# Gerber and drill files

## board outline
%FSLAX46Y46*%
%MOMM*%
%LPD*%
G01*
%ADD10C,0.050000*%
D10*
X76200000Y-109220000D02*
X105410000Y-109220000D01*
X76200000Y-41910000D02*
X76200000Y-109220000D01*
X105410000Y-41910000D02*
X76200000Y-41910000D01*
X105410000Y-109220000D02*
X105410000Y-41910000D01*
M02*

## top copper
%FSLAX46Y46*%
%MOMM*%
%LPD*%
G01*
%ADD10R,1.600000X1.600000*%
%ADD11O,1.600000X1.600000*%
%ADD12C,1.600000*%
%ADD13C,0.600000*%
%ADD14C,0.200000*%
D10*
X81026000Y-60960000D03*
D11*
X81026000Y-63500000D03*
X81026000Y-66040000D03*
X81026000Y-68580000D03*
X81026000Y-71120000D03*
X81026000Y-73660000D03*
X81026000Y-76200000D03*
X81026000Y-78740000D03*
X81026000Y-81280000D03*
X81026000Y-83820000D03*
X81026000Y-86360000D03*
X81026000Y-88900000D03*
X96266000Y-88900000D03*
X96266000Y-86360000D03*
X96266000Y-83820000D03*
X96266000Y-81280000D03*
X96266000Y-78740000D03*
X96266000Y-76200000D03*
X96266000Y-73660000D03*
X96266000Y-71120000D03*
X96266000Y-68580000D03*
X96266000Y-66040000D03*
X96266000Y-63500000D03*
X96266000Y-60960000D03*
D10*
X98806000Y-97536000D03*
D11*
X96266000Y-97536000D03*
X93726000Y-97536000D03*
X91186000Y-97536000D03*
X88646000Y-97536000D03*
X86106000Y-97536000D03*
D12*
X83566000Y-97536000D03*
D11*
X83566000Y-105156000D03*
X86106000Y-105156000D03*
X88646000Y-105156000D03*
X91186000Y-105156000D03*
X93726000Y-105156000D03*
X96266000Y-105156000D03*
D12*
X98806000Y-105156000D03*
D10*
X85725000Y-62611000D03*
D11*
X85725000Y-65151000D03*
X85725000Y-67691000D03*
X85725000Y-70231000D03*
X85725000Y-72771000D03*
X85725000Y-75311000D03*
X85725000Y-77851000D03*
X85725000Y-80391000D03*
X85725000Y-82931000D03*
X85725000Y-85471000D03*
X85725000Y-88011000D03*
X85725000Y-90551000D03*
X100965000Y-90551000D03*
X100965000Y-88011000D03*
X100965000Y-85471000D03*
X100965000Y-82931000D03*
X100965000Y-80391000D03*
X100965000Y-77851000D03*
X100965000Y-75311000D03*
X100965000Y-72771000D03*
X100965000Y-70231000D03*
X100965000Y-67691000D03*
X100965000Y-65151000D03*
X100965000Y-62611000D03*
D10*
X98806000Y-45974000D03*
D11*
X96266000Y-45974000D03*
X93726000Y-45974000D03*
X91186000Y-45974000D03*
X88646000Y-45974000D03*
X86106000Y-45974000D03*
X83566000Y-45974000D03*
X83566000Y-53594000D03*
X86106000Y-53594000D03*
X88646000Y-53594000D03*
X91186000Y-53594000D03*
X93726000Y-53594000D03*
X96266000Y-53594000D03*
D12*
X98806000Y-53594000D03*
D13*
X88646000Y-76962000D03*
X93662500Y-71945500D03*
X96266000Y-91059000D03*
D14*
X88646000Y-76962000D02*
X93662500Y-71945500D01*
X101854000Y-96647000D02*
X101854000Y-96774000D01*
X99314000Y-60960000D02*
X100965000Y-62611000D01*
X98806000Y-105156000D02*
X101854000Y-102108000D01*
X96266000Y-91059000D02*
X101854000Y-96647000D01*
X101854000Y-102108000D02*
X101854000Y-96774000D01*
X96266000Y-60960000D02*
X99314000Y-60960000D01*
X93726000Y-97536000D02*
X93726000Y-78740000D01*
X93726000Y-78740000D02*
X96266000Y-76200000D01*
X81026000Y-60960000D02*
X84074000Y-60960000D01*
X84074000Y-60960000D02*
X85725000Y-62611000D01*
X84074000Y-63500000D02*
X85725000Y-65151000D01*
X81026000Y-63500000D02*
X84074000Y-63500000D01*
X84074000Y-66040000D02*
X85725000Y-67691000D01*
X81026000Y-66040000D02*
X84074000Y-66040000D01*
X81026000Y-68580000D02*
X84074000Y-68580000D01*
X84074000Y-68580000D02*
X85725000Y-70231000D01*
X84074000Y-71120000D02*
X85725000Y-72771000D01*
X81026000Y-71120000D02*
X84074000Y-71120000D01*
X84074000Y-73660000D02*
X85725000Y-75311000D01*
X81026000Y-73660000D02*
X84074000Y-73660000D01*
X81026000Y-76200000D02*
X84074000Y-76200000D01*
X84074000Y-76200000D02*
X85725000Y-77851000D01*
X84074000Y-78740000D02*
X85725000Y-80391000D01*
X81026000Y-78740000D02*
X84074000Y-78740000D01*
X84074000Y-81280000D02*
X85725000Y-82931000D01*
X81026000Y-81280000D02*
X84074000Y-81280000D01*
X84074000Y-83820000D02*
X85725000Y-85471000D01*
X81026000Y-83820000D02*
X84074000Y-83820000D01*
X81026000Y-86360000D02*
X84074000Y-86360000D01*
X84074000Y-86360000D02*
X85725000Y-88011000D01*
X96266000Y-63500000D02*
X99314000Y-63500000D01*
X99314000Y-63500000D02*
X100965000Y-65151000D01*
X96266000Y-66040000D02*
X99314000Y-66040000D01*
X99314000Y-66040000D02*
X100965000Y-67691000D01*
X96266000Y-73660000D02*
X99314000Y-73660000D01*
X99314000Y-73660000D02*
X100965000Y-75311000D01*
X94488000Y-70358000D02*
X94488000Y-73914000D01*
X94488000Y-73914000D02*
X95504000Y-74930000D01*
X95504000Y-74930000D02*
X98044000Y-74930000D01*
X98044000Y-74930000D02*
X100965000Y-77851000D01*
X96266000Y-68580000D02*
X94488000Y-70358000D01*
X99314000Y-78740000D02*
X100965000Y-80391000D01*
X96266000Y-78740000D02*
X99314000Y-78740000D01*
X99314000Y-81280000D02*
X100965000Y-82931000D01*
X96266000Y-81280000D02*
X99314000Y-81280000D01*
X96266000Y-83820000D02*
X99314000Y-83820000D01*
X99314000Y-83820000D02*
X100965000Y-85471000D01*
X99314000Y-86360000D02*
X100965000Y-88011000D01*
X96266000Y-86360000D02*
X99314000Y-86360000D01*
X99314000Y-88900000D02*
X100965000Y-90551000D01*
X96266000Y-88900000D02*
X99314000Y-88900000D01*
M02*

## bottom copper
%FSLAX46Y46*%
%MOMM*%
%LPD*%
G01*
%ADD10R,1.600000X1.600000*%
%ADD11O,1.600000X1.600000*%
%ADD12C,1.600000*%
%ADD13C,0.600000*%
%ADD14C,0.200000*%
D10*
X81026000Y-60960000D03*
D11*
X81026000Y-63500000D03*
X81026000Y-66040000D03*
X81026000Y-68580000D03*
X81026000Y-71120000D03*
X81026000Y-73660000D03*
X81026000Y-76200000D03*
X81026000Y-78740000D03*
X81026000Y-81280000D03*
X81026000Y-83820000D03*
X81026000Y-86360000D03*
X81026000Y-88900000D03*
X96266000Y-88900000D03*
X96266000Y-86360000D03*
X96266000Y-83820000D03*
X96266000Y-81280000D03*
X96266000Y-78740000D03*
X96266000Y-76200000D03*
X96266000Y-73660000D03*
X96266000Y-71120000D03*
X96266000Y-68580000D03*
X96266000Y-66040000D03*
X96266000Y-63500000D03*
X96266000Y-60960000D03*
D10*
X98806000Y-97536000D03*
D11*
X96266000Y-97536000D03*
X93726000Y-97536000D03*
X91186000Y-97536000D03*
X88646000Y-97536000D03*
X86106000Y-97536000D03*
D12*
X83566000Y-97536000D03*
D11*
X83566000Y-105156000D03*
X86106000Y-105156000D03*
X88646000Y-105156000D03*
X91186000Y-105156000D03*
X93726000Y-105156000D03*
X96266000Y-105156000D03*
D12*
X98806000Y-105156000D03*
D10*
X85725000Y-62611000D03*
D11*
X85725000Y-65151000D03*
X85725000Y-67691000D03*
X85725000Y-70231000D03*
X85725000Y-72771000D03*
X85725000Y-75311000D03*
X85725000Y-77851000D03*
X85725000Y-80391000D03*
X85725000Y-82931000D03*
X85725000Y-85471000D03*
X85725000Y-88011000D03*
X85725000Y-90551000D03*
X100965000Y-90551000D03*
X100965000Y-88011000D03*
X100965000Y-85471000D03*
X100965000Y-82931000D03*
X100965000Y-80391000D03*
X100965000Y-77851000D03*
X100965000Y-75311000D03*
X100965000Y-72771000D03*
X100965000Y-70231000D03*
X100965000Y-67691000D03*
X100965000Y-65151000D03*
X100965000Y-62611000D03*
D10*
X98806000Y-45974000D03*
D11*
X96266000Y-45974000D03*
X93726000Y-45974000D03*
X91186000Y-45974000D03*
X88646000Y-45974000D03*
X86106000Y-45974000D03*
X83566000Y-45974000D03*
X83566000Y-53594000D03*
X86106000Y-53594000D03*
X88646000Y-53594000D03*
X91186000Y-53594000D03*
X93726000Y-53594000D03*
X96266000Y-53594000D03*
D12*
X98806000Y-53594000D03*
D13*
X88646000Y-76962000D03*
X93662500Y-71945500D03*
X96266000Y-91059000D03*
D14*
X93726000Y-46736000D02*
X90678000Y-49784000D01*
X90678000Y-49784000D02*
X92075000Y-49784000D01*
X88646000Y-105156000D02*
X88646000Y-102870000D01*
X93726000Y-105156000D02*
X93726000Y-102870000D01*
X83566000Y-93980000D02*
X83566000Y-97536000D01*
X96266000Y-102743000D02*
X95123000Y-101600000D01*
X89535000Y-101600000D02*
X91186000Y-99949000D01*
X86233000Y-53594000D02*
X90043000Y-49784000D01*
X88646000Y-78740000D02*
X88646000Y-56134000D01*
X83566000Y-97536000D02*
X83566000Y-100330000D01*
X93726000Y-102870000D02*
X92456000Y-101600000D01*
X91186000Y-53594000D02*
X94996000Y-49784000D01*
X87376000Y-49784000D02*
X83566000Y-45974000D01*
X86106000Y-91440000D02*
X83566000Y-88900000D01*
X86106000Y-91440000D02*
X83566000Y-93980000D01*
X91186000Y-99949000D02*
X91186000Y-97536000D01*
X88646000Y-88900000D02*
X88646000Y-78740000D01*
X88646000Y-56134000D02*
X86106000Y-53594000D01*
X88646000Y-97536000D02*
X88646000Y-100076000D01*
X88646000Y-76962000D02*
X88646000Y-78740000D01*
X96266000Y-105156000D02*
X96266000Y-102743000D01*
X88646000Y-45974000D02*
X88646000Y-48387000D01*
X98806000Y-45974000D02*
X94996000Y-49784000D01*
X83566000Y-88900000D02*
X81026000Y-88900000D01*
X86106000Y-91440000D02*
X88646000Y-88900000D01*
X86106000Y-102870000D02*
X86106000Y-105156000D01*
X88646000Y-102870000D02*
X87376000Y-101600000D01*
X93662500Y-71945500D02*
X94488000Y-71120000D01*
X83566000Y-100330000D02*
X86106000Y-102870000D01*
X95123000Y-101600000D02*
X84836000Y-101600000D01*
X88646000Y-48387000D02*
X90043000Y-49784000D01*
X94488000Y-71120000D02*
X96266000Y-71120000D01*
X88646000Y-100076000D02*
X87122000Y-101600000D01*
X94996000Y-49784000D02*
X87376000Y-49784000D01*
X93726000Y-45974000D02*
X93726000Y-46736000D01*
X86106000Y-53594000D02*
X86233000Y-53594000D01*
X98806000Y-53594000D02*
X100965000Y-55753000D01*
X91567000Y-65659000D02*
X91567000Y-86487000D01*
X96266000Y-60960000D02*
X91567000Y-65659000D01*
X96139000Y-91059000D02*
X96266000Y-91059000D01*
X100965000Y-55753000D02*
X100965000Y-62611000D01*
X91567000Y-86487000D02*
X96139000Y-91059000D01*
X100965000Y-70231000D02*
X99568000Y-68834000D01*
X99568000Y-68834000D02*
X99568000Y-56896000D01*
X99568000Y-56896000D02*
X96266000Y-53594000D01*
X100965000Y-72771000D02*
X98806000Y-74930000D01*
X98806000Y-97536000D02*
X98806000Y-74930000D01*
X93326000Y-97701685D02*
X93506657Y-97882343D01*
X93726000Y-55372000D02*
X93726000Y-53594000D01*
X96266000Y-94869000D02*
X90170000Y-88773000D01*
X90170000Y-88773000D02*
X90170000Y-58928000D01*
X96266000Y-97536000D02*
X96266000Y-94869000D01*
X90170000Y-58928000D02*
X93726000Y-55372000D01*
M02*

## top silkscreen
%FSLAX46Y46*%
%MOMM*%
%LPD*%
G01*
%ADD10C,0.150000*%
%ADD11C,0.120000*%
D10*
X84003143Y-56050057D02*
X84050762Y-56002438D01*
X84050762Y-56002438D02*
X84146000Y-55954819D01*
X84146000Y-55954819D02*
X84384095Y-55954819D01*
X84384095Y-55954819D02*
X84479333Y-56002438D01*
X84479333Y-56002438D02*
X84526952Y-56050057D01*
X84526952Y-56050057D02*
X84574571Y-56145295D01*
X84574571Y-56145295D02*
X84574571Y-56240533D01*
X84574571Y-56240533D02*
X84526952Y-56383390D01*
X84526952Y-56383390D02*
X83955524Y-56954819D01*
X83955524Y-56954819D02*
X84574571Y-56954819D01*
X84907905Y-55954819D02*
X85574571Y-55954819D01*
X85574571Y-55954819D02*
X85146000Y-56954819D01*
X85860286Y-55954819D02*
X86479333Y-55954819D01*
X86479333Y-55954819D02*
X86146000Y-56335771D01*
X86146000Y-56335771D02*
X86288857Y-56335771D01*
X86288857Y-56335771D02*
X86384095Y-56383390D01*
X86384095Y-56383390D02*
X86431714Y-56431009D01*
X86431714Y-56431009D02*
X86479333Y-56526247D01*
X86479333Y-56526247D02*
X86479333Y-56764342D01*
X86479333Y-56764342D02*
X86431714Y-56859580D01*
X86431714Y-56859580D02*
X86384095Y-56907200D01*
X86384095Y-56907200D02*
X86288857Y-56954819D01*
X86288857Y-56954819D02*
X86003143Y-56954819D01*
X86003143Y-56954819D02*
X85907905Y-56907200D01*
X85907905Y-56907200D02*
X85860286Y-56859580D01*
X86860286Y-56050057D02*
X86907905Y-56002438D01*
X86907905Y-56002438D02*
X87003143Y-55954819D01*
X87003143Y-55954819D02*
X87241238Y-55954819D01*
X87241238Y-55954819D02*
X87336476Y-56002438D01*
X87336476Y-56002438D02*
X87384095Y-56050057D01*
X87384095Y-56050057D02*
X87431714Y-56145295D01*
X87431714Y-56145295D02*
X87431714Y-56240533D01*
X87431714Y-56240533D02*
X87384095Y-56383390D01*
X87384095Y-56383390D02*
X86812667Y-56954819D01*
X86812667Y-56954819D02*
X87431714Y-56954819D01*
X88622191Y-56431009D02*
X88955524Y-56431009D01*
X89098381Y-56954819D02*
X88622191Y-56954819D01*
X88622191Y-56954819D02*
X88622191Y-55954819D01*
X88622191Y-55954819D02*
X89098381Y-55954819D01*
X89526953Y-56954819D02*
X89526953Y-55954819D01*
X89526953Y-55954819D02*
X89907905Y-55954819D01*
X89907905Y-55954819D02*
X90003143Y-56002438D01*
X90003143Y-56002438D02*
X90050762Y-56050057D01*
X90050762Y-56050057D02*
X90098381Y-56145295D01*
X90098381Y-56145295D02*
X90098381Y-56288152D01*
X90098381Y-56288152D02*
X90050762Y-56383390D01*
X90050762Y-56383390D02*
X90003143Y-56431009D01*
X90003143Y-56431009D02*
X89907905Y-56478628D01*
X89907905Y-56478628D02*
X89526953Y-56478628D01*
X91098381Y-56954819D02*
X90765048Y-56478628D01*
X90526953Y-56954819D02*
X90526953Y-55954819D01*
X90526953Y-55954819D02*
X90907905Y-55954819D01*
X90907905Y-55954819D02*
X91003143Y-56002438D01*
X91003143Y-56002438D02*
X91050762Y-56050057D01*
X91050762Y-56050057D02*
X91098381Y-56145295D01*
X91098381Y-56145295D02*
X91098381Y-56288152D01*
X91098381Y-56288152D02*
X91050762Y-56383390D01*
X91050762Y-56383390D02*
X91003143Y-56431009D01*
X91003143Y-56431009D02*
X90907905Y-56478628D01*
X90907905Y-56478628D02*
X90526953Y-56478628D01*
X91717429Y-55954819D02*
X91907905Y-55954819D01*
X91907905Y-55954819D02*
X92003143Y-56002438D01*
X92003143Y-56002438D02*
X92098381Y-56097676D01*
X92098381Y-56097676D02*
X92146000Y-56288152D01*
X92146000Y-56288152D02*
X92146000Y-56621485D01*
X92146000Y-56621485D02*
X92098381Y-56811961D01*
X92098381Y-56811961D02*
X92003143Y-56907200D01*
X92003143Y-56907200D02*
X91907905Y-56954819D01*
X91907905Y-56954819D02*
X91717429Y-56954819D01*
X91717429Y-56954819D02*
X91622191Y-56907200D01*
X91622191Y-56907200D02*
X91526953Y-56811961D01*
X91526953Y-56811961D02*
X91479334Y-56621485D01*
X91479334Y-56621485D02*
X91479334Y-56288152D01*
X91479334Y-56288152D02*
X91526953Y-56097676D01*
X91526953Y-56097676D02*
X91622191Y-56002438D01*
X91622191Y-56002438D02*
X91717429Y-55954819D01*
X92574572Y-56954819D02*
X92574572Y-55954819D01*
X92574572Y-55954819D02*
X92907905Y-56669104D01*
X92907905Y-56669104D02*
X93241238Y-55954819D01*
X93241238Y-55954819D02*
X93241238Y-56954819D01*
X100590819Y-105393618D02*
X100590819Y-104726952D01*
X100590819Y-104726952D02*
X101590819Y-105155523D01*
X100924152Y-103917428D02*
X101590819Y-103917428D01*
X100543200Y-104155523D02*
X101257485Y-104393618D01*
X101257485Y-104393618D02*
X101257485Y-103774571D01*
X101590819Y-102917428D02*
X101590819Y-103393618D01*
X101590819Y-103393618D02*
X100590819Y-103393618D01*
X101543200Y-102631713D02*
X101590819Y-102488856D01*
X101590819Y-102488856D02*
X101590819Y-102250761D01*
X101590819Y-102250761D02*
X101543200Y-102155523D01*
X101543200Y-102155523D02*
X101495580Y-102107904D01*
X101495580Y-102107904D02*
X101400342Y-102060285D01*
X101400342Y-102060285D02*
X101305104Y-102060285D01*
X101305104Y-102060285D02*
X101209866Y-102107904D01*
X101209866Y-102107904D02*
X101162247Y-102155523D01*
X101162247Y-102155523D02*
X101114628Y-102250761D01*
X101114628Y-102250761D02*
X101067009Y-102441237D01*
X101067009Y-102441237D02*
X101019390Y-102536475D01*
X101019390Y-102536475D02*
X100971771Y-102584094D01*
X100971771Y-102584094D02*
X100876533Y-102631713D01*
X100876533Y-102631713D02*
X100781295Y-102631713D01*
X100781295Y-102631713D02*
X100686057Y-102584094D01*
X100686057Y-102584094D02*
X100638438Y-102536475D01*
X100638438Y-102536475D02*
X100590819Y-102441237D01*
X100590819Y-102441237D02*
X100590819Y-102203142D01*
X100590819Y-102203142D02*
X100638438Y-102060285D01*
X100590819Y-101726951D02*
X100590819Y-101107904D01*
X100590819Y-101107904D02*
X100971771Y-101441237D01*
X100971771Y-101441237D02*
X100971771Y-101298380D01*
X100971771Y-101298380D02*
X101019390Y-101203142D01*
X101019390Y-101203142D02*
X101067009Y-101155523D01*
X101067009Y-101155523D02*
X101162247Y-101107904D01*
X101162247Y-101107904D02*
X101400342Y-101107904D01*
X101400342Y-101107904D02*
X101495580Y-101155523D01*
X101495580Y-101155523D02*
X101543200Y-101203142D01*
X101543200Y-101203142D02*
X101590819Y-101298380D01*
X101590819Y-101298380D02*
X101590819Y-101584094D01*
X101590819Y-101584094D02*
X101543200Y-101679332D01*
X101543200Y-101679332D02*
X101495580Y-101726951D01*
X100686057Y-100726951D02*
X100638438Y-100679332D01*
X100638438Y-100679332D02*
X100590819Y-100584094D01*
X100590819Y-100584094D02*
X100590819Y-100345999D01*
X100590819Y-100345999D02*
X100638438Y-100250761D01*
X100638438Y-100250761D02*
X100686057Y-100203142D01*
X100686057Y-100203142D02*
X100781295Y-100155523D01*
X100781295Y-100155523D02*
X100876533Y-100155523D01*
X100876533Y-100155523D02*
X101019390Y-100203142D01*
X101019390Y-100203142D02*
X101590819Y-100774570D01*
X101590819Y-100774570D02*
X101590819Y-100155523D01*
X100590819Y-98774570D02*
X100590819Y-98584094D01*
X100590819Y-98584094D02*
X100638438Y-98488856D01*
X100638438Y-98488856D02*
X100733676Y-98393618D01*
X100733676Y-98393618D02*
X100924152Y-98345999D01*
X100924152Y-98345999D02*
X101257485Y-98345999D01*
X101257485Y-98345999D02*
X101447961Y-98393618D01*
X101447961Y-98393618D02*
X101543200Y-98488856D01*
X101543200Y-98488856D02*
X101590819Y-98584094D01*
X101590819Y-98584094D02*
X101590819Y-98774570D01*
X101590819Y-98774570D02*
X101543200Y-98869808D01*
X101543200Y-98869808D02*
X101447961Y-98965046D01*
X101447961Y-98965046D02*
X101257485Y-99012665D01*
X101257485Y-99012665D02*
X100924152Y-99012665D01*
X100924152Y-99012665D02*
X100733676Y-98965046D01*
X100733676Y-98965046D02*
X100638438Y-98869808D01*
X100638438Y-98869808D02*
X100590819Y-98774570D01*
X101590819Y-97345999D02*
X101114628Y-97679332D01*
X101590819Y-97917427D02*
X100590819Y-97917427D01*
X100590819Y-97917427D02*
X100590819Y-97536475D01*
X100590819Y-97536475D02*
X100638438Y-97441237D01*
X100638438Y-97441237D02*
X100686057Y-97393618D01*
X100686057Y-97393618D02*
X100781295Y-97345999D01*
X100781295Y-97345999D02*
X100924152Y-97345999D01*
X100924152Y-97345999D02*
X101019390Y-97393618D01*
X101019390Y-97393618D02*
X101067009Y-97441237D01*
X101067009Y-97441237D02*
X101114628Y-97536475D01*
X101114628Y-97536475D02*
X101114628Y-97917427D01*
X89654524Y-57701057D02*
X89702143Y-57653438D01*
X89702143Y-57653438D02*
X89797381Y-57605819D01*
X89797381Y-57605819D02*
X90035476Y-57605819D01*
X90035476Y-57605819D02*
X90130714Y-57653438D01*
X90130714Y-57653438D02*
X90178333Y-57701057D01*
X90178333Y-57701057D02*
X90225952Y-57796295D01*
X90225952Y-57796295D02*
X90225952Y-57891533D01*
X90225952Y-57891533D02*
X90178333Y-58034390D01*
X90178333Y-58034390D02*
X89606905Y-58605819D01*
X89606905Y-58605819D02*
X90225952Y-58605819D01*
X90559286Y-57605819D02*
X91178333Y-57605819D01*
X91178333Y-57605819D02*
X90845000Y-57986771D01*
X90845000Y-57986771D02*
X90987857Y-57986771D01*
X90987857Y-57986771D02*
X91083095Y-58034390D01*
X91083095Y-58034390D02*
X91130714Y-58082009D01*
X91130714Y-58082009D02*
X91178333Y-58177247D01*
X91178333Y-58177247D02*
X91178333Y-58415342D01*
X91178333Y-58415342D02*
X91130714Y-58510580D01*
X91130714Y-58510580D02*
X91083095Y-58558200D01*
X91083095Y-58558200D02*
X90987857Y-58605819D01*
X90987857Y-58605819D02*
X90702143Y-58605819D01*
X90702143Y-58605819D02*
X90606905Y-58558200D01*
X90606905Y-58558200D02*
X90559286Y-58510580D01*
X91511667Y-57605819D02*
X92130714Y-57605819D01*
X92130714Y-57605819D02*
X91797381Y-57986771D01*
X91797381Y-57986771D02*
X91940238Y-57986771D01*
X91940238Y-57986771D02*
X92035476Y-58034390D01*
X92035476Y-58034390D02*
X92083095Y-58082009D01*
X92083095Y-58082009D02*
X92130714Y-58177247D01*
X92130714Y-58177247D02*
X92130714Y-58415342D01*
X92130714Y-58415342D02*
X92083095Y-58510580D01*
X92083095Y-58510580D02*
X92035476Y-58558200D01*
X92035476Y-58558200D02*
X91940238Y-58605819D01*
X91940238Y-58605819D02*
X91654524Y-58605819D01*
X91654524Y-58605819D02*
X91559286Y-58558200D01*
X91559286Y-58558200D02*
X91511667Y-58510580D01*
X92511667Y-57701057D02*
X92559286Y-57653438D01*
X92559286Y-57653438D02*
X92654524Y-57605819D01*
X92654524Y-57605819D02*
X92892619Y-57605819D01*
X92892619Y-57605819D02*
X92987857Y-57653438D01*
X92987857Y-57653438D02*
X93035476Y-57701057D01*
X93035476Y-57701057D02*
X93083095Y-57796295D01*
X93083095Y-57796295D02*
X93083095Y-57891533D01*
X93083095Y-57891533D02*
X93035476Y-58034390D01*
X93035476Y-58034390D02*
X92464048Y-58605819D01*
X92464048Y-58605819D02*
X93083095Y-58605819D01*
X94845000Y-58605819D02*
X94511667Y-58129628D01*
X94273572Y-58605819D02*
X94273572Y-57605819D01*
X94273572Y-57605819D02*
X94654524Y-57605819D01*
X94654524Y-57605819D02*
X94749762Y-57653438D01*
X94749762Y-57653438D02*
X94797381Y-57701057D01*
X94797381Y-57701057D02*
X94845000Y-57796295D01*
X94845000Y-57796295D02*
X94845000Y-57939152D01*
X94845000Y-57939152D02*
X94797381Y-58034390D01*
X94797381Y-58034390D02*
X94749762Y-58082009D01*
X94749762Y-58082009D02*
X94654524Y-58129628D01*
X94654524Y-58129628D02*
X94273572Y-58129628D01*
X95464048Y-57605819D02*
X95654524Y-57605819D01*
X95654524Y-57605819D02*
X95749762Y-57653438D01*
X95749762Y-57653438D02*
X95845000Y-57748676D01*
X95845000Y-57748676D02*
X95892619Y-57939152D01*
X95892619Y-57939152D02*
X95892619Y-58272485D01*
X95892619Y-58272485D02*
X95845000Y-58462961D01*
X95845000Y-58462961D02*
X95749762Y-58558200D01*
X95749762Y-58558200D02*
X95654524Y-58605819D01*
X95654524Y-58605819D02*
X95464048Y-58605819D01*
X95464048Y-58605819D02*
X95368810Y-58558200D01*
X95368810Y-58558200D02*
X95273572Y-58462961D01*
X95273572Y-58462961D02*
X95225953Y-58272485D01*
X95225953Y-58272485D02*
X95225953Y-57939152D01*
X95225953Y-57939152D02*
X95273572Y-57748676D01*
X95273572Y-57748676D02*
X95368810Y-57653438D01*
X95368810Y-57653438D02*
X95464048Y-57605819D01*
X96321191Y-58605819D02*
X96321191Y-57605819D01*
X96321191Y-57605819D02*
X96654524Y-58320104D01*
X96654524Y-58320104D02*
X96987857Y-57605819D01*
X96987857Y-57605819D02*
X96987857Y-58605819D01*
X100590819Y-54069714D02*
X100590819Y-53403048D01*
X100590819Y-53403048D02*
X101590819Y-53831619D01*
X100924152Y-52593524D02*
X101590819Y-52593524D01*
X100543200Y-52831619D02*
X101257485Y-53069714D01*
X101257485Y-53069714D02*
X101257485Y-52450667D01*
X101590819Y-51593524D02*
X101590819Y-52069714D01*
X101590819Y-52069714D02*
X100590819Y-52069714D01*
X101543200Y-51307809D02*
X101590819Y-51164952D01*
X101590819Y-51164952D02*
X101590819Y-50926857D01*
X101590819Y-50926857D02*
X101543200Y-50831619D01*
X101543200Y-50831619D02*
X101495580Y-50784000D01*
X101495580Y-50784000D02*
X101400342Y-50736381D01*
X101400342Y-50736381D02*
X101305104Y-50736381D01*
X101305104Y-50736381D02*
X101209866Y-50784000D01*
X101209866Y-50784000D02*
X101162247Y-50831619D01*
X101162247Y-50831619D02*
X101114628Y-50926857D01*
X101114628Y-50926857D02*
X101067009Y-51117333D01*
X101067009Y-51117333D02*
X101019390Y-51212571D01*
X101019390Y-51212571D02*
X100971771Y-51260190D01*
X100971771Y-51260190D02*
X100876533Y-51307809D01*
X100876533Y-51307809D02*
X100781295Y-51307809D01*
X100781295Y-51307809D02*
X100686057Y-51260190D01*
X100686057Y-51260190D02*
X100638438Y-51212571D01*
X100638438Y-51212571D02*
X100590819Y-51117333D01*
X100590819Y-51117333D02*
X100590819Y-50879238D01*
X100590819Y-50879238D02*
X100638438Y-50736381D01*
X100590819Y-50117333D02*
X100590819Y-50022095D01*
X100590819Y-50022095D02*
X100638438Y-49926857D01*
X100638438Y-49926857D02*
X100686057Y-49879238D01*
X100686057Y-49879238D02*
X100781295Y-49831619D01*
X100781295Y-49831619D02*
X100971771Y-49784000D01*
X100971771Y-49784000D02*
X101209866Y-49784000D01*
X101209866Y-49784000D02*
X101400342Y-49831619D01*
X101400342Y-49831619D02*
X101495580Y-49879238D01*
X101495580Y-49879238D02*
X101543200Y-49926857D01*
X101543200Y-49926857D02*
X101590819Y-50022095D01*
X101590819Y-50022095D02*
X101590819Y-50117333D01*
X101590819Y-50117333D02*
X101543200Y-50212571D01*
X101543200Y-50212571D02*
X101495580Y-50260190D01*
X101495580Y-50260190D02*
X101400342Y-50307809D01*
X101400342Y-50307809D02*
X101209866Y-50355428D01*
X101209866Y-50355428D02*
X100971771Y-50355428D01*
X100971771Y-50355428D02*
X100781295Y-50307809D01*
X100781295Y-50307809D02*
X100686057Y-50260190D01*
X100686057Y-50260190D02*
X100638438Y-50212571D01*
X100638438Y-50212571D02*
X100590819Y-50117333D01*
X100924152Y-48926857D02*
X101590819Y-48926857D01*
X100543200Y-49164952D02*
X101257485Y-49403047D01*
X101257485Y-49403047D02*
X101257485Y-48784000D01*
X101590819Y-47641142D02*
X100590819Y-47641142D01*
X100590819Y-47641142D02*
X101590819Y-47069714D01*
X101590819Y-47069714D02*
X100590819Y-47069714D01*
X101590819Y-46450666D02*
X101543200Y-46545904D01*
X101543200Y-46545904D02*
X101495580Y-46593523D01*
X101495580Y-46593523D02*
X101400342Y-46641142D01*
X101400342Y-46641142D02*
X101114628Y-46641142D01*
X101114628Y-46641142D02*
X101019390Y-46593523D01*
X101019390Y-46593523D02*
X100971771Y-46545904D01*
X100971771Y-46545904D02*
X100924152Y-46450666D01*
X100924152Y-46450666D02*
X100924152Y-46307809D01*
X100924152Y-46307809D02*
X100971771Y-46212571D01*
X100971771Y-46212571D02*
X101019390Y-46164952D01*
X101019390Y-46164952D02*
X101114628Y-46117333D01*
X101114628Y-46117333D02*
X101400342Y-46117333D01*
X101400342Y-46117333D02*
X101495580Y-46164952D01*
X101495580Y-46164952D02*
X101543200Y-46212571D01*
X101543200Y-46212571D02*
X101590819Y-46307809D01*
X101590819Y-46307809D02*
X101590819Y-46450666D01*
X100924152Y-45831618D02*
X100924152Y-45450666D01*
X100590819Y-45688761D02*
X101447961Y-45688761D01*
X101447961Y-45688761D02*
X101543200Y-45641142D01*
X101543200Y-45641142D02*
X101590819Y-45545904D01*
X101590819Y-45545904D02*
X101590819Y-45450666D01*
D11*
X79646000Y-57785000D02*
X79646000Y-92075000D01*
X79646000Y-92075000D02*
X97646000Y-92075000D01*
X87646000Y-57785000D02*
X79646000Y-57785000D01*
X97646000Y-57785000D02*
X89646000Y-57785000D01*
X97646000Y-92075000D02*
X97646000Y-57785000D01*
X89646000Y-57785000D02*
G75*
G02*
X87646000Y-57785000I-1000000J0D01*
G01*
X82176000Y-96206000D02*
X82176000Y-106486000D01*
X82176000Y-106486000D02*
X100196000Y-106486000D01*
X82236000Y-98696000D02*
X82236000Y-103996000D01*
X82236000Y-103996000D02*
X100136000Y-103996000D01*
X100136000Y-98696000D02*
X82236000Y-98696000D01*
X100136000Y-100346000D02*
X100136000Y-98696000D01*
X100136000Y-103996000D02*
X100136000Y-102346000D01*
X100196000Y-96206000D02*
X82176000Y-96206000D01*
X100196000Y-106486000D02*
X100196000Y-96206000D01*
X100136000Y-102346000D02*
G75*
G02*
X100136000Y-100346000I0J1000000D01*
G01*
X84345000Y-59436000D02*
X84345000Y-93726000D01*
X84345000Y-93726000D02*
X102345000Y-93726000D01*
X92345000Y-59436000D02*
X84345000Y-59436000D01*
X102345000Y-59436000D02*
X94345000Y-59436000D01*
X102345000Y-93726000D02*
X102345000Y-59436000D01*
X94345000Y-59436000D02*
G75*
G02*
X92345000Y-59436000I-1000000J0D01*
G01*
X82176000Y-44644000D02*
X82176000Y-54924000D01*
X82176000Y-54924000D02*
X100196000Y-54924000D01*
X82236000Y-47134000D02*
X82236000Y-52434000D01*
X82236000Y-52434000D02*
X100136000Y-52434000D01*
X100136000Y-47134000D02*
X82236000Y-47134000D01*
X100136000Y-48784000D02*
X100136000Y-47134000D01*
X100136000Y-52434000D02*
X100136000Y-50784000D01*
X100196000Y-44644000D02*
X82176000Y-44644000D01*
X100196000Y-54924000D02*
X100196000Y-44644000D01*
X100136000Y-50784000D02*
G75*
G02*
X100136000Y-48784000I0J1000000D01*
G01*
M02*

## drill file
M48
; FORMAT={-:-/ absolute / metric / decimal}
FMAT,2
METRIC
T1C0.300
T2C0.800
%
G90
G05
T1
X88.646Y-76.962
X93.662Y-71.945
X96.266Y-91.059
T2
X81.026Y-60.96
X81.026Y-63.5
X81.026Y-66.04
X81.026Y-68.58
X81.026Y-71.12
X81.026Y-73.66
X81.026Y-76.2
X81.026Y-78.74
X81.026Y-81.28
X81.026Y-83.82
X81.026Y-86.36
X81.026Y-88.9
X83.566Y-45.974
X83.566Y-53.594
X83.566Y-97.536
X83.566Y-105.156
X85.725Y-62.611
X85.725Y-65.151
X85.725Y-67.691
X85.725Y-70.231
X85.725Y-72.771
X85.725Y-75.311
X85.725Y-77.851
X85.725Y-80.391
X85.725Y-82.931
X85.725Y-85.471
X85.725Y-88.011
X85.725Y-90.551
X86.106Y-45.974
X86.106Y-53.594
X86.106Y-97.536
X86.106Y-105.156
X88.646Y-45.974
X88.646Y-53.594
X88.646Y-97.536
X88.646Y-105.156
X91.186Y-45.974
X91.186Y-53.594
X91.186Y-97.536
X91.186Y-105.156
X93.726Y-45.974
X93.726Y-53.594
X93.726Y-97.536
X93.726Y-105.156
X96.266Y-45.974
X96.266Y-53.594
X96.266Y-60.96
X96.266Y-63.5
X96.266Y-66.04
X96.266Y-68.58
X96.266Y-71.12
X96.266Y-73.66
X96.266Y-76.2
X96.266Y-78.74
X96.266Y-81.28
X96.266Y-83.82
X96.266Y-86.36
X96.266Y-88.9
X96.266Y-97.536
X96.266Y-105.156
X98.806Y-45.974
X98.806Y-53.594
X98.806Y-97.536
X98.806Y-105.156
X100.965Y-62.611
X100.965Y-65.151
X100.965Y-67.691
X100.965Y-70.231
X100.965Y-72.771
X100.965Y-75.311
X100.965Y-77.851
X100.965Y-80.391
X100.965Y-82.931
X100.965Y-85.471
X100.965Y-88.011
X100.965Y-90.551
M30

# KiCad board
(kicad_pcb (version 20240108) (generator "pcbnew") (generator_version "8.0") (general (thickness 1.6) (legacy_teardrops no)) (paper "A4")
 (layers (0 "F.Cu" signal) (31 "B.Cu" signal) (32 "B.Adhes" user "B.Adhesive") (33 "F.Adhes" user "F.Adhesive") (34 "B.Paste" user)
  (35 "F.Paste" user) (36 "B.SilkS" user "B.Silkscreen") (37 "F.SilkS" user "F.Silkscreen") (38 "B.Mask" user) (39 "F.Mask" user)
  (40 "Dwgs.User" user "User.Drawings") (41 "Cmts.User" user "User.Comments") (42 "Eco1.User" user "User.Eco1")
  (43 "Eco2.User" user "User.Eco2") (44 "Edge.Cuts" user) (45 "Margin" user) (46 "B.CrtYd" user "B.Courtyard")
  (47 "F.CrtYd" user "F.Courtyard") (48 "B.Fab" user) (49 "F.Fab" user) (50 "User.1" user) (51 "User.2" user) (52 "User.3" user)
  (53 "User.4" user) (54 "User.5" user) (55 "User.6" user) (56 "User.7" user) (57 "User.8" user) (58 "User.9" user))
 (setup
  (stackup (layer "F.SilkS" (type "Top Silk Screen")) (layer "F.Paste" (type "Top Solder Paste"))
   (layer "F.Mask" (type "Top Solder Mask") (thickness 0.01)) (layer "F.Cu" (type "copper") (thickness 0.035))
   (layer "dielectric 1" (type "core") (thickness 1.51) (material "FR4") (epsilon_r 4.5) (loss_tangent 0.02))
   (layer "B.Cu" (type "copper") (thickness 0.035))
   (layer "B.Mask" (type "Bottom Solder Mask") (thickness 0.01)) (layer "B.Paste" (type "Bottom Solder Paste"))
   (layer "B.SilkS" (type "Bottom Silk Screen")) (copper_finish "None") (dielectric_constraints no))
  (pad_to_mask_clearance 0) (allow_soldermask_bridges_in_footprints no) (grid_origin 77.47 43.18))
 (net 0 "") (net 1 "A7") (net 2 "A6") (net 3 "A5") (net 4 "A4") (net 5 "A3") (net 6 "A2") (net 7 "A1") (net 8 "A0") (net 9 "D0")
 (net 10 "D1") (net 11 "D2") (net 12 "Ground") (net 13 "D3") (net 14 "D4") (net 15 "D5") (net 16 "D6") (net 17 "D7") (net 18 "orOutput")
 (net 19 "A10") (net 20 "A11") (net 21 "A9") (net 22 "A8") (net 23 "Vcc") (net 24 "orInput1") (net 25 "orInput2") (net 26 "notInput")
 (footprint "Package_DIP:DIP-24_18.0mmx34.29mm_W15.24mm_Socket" (layer "F.Cu") (at 81.026 60.96)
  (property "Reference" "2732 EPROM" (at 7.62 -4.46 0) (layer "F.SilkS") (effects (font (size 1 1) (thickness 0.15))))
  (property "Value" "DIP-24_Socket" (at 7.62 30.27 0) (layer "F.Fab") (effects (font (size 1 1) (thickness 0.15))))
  (fp_line (start -1.38 -3.175) (end -1.38 31.115) (stroke (width 0.12) (type solid)) (layer "F.SilkS"))
  (fp_line (start -1.38 31.115) (end 16.62 31.115) (stroke (width 0.12) (type solid)) (layer "F.SilkS"))
  (fp_line (start 6.62 -3.175) (end -1.38 -3.175) (stroke (width 0.12) (type solid)) (layer "F.SilkS"))
  (fp_line (start 16.62 -3.175) (end 8.62 -3.175) (stroke (width 0.12) (type solid)) (layer "F.SilkS"))
  (fp_line (start 16.62 31.115) (end 16.62 -3.175) (stroke (width 0.12) (type solid)) (layer "F.SilkS"))
  (fp_arc (start 8.62 -3.175) (mid 7.62 -2.175) (end 6.62 -3.175) (stroke (width 0.12) (type solid)) (layer "F.SilkS"))
  (pad "1" thru_hole rect (at 0 0) (size 1.6 1.6) (drill 0.8) (layers "*.Cu" "*.Mask") (remove_unused_layers no) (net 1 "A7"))
  (pad "2" thru_hole oval (at 0 2.54) (size 1.6 1.6) (drill 0.8) (layers "*.Cu" "*.Mask") (remove_unused_layers no) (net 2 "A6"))
  (pad "3" thru_hole oval (at 0 5.08) (size 1.6 1.6) (drill 0.8) (layers "*.Cu" "*.Mask") (remove_unused_layers no) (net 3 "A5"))
  (pad "4" thru_hole oval (at 0 7.62) (size 1.6 1.6) (drill 0.8) (layers "*.Cu" "*.Mask") (remove_unused_layers no) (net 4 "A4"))
  (pad "5" thru_hole oval (at 0 10.16) (size 1.6 1.6) (drill 0.8) (layers "*.Cu" "*.Mask") (remove_unused_layers no) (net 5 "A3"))
  (pad "6" thru_hole oval (at 0 12.7) (size 1.6 1.6) (drill 0.8) (layers "*.Cu" "*.Mask") (remove_unused_layers no) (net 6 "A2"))
  (pad "7" thru_hole oval (at 0 15.24) (size 1.6 1.6) (drill 0.8) (layers "*.Cu" "*.Mask") (remove_unused_layers no) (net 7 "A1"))
  (pad "8" thru_hole oval (at 0 17.78) (size 1.6 1.6) (drill 0.8) (layers "*.Cu" "*.Mask") (remove_unused_layers no) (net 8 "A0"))
  (pad "9" thru_hole oval (at 0 20.32) (size 1.6 1.6) (drill 0.8) (layers "*.Cu" "*.Mask") (remove_unused_layers no) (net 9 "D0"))
  (pad "10" thru_hole oval (at 0 22.86) (size 1.6 1.6) (drill 0.8) (layers "*.Cu" "*.Mask") (remove_unused_layers no) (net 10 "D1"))
  (pad "11" thru_hole oval (at 0 25.4) (size 1.6 1.6) (drill 0.8) (layers "*.Cu" "*.Mask") (remove_unused_layers no) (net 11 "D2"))
  (pad "12" thru_hole oval (at 0 27.94) (size 1.6 1.6) (drill 0.8) (layers "*.Cu" "*.Mask") (remove_unused_layers no) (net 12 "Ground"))
  (pad "13" thru_hole oval (at 15.24 27.94) (size 1.6 1.6) (drill 0.8) (layers "*.Cu" "*.Mask") (remove_unused_layers no) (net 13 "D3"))
  (pad "14" thru_hole oval (at 15.24 25.4) (size 1.6 1.6) (drill 0.8) (layers "*.Cu" "*.Mask") (remove_unused_layers no) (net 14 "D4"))
  (pad "15" thru_hole oval (at 15.24 22.86) (size 1.6 1.6) (drill 0.8) (layers "*.Cu" "*.Mask") (remove_unused_layers no) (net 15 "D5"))
  (pad "16" thru_hole oval (at 15.24 20.32) (size 1.6 1.6) (drill 0.8) (layers "*.Cu" "*.Mask") (remove_unused_layers no) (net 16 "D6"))
  (pad "17" thru_hole oval (at 15.24 17.78) (size 1.6 1.6) (drill 0.8) (layers "*.Cu" "*.Mask") (remove_unused_layers no) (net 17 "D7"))
  (pad "18" thru_hole oval (at 15.24 15.24) (size 1.6 1.6) (drill 0.8) (layers "*.Cu" "*.Mask") (remove_unused_layers no)
   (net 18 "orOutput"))
  (pad "19" thru_hole oval (at 15.24 12.7) (size 1.6 1.6) (drill 0.8) (layers "*.Cu" "*.Mask") (remove_unused_layers no) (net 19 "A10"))
  (pad "20" thru_hole oval (at 15.24 10.16) (size 1.6 1.6) (drill 0.8) (layers "*.Cu" "*.Mask") (remove_unused_layers no) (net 12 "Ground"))
  (pad "21" thru_hole oval (at 15.24 7.62) (size 1.6 1.6) (drill 0.8) (layers "*.Cu" "*.Mask") (remove_unused_layers no) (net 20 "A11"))
  (pad "22" thru_hole oval (at 15.24 5.08) (size 1.6 1.6) (drill 0.8) (layers "*.Cu" "*.Mask") (remove_unused_layers no) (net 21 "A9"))
  (pad "23" thru_hole oval (at 15.24 2.54) (size 1.6 1.6) (drill 0.8) (layers "*.Cu" "*.Mask") (remove_unused_layers no) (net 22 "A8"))
  (pad "24" thru_hole oval (at 15.24 0) (size 1.6 1.6) (drill 0.8) (layers "*.Cu" "*.Mask") (remove_unused_layers no) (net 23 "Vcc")))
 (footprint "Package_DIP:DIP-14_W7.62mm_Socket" (layer "F.Cu") (at 98.806 97.536 -90)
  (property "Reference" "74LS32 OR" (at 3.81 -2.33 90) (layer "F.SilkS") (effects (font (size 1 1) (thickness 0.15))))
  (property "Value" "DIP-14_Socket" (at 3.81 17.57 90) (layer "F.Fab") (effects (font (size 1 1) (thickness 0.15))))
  (fp_line (start -1.33 16.63) (end 8.95 16.63) (stroke (width 0.12) (type solid)) (layer "F.SilkS"))
  (fp_line (start 8.95 16.63) (end 8.95 -1.39) (stroke (width 0.12) (type solid)) (layer "F.SilkS"))
  (fp_line (start 1.16 16.57) (end 6.46 16.57) (stroke (width 0.12) (type solid)) (layer "F.SilkS"))
  (fp_line (start 6.46 16.57) (end 6.46 -1.33) (stroke (width 0.12) (type solid)) (layer "F.SilkS"))
  (fp_line (start 1.16 -1.33) (end 1.16 16.57) (stroke (width 0.12) (type solid)) (layer "F.SilkS"))
  (fp_line (start 2.81 -1.33) (end 1.16 -1.33) (stroke (width 0.12) (type solid)) (layer "F.SilkS"))
  (fp_line (start 6.46 -1.33) (end 4.81 -1.33) (stroke (width 0.12) (type solid)) (layer "F.SilkS"))
  (fp_line (start -1.33 -1.39) (end -1.33 16.63) (stroke (width 0.12) (type solid)) (layer "F.SilkS"))
  (fp_line (start 8.95 -1.39) (end -1.33 -1.39) (stroke (width 0.12) (type solid)) (layer "F.SilkS"))
  (fp_arc (start 4.81 -1.33) (mid 3.81 -0.33) (end 2.81 -1.33) (stroke (width 0.12) (type solid)) (layer "F.SilkS"))
  (pad "1" thru_hole rect (at 0 0 270) (size 1.6 1.6) (drill 0.8) (layers "*.Cu" "*.Mask") (remove_unused_layers no) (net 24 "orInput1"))
  (pad "2" thru_hole oval (at 0 2.54 270) (size 1.6 1.6) (drill 0.8) (layers "*.Cu" "*.Mask") (remove_unused_layers no) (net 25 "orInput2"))
  (pad "3" thru_hole oval (at 0 5.08 270) (size 1.6 1.6) (drill 0.8) (layers "*.Cu" "*.Mask") (remove_unused_layers no) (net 18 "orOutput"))
  (pad "4" thru_hole oval (at 0 7.62 270) (size 1.6 1.6) (drill 0.8) (layers "*.Cu" "*.Mask") (remove_unused_layers no) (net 12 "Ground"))
  (pad "5" thru_hole oval (at 0 10.16 270) (size 1.6 1.6) (drill 0.8) (layers "*.Cu" "*.Mask") (remove_unused_layers no) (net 12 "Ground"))
  (pad "6" thru_hole oval (at 0 12.7 270) (size 1.6 1.6) (drill 0.8) (layers "*.Cu" "*.Mask") (remove_unused_layers no))
  (pad "7" thru_hole circle (at 0 15.24 270) (size 1.6 1.6) (drill 0.8) (layers "*.Cu" "*.Mask") (remove_unused_layers no) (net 12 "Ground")
   (thermal_bridge_angle 90))
  (pad "8" thru_hole oval (at 7.62 15.24 270) (size 1.6 1.6) (drill 0.8) (layers "*.Cu" "*.Mask") (remove_unused_layers no))
  (pad "9" thru_hole oval (at 7.62 12.7 270) (size 1.6 1.6) (drill 0.8) (layers "*.Cu" "*.Mask") (remove_unused_layers no) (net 12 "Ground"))
  (pad "10" thru_hole oval (at 7.62 10.16 270) (size 1.6 1.6) (drill 0.8) (layers "*.Cu" "*.Mask") (remove_unused_layers no)
   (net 12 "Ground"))
  (pad "11" thru_hole oval (at 7.62 7.62 270) (size 1.6 1.6) (drill 0.8) (layers "*.Cu" "*.Mask") (remove_unused_layers no))
  (pad "12" thru_hole oval (at 7.62 5.08 270) (size 1.6 1.6) (drill 0.8) (layers "*.Cu" "*.Mask") (remove_unused_layers no)
   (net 12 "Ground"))
  (pad "13" thru_hole oval (at 7.62 2.54 270) (size 1.6 1.6) (drill 0.8) (layers "*.Cu" "*.Mask") (remove_unused_layers no)
   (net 12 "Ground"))
  (pad "14" thru_hole circle (at 7.62 0 270) (size 1.6 1.6) (drill 0.8) (layers "*.Cu" "*.Mask") (remove_unused_layers no) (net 23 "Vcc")
   (thermal_bridge_angle 90)))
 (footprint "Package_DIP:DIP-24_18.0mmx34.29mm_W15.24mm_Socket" (layer "F.Cu") (at 85.725 62.611)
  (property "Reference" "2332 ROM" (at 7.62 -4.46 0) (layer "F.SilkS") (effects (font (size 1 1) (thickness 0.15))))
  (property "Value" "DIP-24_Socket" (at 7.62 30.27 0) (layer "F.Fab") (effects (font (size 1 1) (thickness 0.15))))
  (fp_line (start -1.38 -3.175) (end -1.38 31.115) (stroke (width 0.12) (type solid)) (layer "F.SilkS"))
  (fp_line (start -1.38 31.115) (end 16.62 31.115) (stroke (width 0.12) (type solid)) (layer "F.SilkS"))
  (fp_line (start 6.62 -3.175) (end -1.38 -3.175) (stroke (width 0.12) (type solid)) (layer "F.SilkS"))
  (fp_line (start 16.62 -3.175) (end 8.62 -3.175) (stroke (width 0.12) (type solid)) (layer "F.SilkS"))
  (fp_line (start 16.62 31.115) (end 16.62 -3.175) (stroke (width 0.12) (type solid)) (layer "F.SilkS"))
  (fp_arc (start 8.62 -3.175) (mid 7.62 -2.175) (end 6.62 -3.175) (stroke (width 0.12) (type solid)) (layer "F.SilkS"))
  (pad "1" thru_hole rect (at 0 0) (size 1.6 1.6) (drill 0.8) (layers "*.Cu" "*.Mask") (remove_unused_layers no) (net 1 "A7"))
  (pad "2" thru_hole oval (at 0 2.54) (size 1.6 1.6) (drill 0.8) (layers "*.Cu" "*.Mask") (remove_unused_layers no) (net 2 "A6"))
  (pad "3" thru_hole oval (at 0 5.08) (size 1.6 1.6) (drill 0.8) (layers "*.Cu" "*.Mask") (remove_unused_layers no) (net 3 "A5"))
  (pad "4" thru_hole oval (at 0 7.62) (size 1.6 1.6) (drill 0.8) (layers "*.Cu" "*.Mask") (remove_unused_layers no) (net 4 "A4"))
  (pad "5" thru_hole oval (at 0 10.16) (size 1.6 1.6) (drill 0.8) (layers "*.Cu" "*.Mask") (remove_unused_layers no) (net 5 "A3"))
  (pad "6" thru_hole oval (at 0 12.7) (size 1.6 1.6) (drill 0.8) (layers "*.Cu" "*.Mask") (remove_unused_layers no) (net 6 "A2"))
  (pad "7" thru_hole oval (at 0 15.24) (size 1.6 1.6) (drill 0.8) (layers "*.Cu" "*.Mask") (remove_unused_layers no) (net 7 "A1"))
  (pad "8" thru_hole oval (at 0 17.78) (size 1.6 1.6) (drill 0.8) (layers "*.Cu" "*.Mask") (remove_unused_layers no) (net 8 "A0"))
  (pad "9" thru_hole oval (at 0 20.32) (size 1.6 1.6) (drill 0.8) (layers "*.Cu" "*.Mask") (remove_unused_layers no) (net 9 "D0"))
  (pad "10" thru_hole oval (at 0 22.86) (size 1.6 1.6) (drill 0.8) (layers "*.Cu" "*.Mask") (remove_unused_layers no) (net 10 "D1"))
  (pad "11" thru_hole oval (at 0 25.4) (size 1.6 1.6) (drill 0.8) (layers "*.Cu" "*.Mask") (remove_unused_layers no) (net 11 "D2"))
  (pad "12" thru_hole oval (at 0 27.94) (size 1.6 1.6) (drill 0.8) (layers "*.Cu" "*.Mask") (remove_unused_layers no) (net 12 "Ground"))
  (pad "13" thru_hole oval (at 15.24 27.94) (size 1.6 1.6) (drill 0.8) (layers "*.Cu" "*.Mask") (remove_unused_layers no) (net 13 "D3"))
  (pad "14" thru_hole oval (at 15.24 25.4) (size 1.6 1.6) (drill 0.8) (layers "*.Cu" "*.Mask") (remove_unused_layers no) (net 14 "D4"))
  (pad "15" thru_hole oval (at 15.24 22.86) (size 1.6 1.6) (drill 0.8) (layers "*.Cu" "*.Mask") (remove_unused_layers no) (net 15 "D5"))
  (pad "16" thru_hole oval (at 15.24 20.32) (size 1.6 1.6) (drill 0.8) (layers "*.Cu" "*.Mask") (remove_unused_layers no) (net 16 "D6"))
  (pad "17" thru_hole oval (at 15.24 17.78) (size 1.6 1.6) (drill 0.8) (layers "*.Cu" "*.Mask") (remove_unused_layers no) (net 17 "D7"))
  (pad "18" thru_hole oval (at 15.24 15.24) (size 1.6 1.6) (drill 0.8) (layers "*.Cu" "*.Mask") (remove_unused_layers no) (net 20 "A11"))
  (pad "19" thru_hole oval (at 15.24 12.7) (size 1.6 1.6) (drill 0.8) (layers "*.Cu" "*.Mask") (remove_unused_layers no) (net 19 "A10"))
  (pad "20" thru_hole oval (at 15.24 10.16) (size 1.6 1.6) (drill 0.8) (layers "*.Cu" "*.Mask") (remove_unused_layers no)
   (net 24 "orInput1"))
  (pad "21" thru_hole oval (at 15.24 7.62) (size 1.6 1.6) (drill 0.8) (layers "*.Cu" "*.Mask") (remove_unused_layers no) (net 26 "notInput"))
  (pad "22" thru_hole oval (at 15.24 5.08) (size 1.6 1.6) (drill 0.8) (layers "*.Cu" "*.Mask") (remove_unused_layers no) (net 21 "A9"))
  (pad "23" thru_hole oval (at 15.24 2.54) (size 1.6 1.6) (drill 0.8) (layers "*.Cu" "*.Mask") (remove_unused_layers no) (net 22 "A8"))
  (pad "24" thru_hole oval (at 15.24 0) (size 1.6 1.6) (drill 0.8) (layers "*.Cu" "*.Mask") (remove_unused_layers no) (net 23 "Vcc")))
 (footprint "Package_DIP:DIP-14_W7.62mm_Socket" (layer "F.Cu") (at 98.806 45.974 -90)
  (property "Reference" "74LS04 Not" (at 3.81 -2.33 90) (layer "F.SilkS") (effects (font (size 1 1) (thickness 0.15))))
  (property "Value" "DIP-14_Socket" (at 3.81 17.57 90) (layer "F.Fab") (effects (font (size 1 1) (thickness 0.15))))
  (fp_line (start -1.33 16.63) (end 8.95 16.63) (stroke (width 0.12) (type solid)) (layer "F.SilkS"))
  (fp_line (start 8.95 16.63) (end 8.95 -1.39) (stroke (width 0.12) (type solid)) (layer "F.SilkS"))
  (fp_line (start 1.16 16.57) (end 6.46 16.57) (stroke (width 0.12) (type solid)) (layer "F.SilkS"))
  (fp_line (start 6.46 16.57) (end 6.46 -1.33) (stroke (width 0.12) (type solid)) (layer "F.SilkS"))
  (fp_line (start 1.16 -1.33) (end 1.16 16.57) (stroke (width 0.12) (type solid)) (layer "F.SilkS"))
  (fp_line (start 2.81 -1.33) (end 1.16 -1.33) (stroke (width 0.12) (type solid)) (layer "F.SilkS"))
  (fp_line (start 6.46 -1.33) (end 4.81 -1.33) (stroke (width 0.12) (type solid)) (layer "F.SilkS"))
  (fp_line (start -1.33 -1.39) (end -1.33 16.63) (stroke (width 0.12) (type solid)) (layer "F.SilkS"))
  (fp_line (start 8.95 -1.39) (end -1.33 -1.39) (stroke (width 0.12) (type solid)) (layer "F.SilkS"))
  (fp_arc (start 4.81 -1.33) (mid 3.81 -0.33) (end 2.81 -1.33) (stroke (width 0.12) (type solid)) (layer "F.SilkS"))
  (pad "1" thru_hole rect (at 0 0 270) (size 1.6 1.6) (drill 0.8) (layers "*.Cu" "*.Mask") (remove_unused_layers no) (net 12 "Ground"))
  (pad "2" thru_hole oval (at 0 2.54 270) (size 1.6 1.6) (drill 0.8) (layers "*.Cu" "*.Mask") (remove_unused_layers no))
  (pad "3" thru_hole oval (at 0 5.08 270) (size 1.6 1.6) (drill 0.8) (layers "*.Cu" "*.Mask") (remove_unused_layers no) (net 12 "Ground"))
  (pad "4" thru_hole oval (at 0 7.62 270) (size 1.6 1.6) (drill 0.8) (layers "*.Cu" "*.Mask") (remove_unused_layers no))
  (pad "5" thru_hole oval (at 0 10.16 270) (size 1.6 1.6) (drill 0.8) (layers "*.Cu" "*.Mask") (remove_unused_layers no) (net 12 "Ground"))
  (pad "6" thru_hole oval (at 0 12.7 270) (size 1.6 1.6) (drill 0.8) (layers "*.Cu" "*.Mask") (remove_unused_layers no))
  (pad "7" thru_hole oval (at 0 15.24 270) (size 1.6 1.6) (drill 0.8) (layers "*.Cu" "*.Mask") (remove_unused_layers no) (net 12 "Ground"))
  (pad "8" thru_hole oval (at 7.62 15.24 270) (size 1.6 1.6) (drill 0.8) (layers "*.Cu" "*.Mask") (remove_unused_layers no))
  (pad "9" thru_hole oval (at 7.62 12.7 270) (size 1.6 1.6) (drill 0.8) (layers "*.Cu" "*.Mask") (remove_unused_layers no) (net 12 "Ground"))
  (pad "10" thru_hole oval (at 7.62 10.16 270) (size 1.6 1.6) (drill 0.8) (layers "*.Cu" "*.Mask") (remove_unused_layers no))
  (pad "11" thru_hole oval (at 7.62 7.62 270) (size 1.6 1.6) (drill 0.8) (layers "*.Cu" "*.Mask") (remove_unused_layers no)
   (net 12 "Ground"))
  (pad "12" thru_hole oval (at 7.62 5.08 270) (size 1.6 1.6) (drill 0.8) (layers "*.Cu" "*.Mask") (remove_unused_layers no)
   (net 25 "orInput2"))
  (pad "13" thru_hole oval (at 7.62 2.54 270) (size 1.6 1.6) (drill 0.8) (layers "*.Cu" "*.Mask") (remove_unused_layers no)
   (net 26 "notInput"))
  (pad "14" thru_hole circle (at 7.62 0 270) (size 1.6 1.6) (drill 0.8) (layers "*.Cu" "*.Mask") (remove_unused_layers no) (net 23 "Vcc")
   (thermal_bridge_angle 90)))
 (gr_line (start 76.2 109.22) (end 105.41 109.22) (stroke (width 0.05) (type default)) (layer "Edge.Cuts"))
 (gr_line (start 76.2 41.91) (end 76.2 109.22) (stroke (width 0.05) (type default)) (layer "Edge.Cuts"))
 (gr_line (start 105.41 41.91) (end 76.2 41.91) (stroke (width 0.05) (type default)) (layer "Edge.Cuts"))
 (gr_line (start 105.41 109.22) (end 105.41 41.91) (stroke (width 0.05) (type default)) (layer "Edge.Cuts"))
 (segment (start 88.646 76.962) (end 93.6625 71.9455) (width 0.2) (layer "F.Cu") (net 12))
 (via (at 88.646 76.962) (size 0.6) (drill 0.3) (layers "F.Cu" "B.Cu") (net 12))
 (via (at 93.6625 71.9455) (size 0.6) (drill 0.3) (layers "F.Cu" "B.Cu") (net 12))
 (segment (start 93.726 46.736) (end 90.678 49.784) (width 0.2) (layer "B.Cu") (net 12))
 (segment (start 90.678 49.784) (end 92.075 49.784) (width 0.2) (layer "B.Cu") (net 12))
 (segment (start 88.646 105.156) (end 88.646 102.87) (width 0.2) (layer "B.Cu") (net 12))
 (segment (start 93.726 105.156) (end 93.726 102.87) (width 0.2) (layer "B.Cu") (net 12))
 (segment (start 83.566 93.98) (end 83.566 97.536) (width 0.2) (layer "B.Cu") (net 12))
 (segment (start 96.266 102.743) (end 95.123 101.6) (width 0.2) (layer "B.Cu") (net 12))
 (segment (start 89.535 101.6) (end 91.186 99.949) (width 0.2) (layer "B.Cu") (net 12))
 (segment (start 86.233 53.594) (end 90.043 49.784) (width 0.2) (layer "B.Cu") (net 12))
 (segment (start 88.646 78.74) (end 88.646 56.134) (width 0.2) (layer "B.Cu") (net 12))
 (segment (start 83.566 97.536) (end 83.566 100.33) (width 0.2) (layer "B.Cu") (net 12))
 (segment (start 93.726 102.87) (end 92.456 101.6) (width 0.2) (layer "B.Cu") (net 12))
 (segment (start 91.186 53.594) (end 94.996 49.784) (width 0.2) (layer "B.Cu") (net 12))
 (segment (start 87.376 49.784) (end 83.566 45.974) (width 0.2) (layer "B.Cu") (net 12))
 (segment (start 86.106 91.44) (end 83.566 88.9) (width 0.2) (layer "B.Cu") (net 12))
 (segment (start 86.106 91.44) (end 83.566 93.98) (width 0.2) (layer "B.Cu") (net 12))
 (segment (start 91.186 99.949) (end 91.186 97.536) (width 0.2) (layer "B.Cu") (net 12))
 (segment (start 88.646 88.9) (end 88.646 78.74) (width 0.2) (layer "B.Cu") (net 12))
 (segment (start 88.646 56.134) (end 86.106 53.594) (width 0.2) (layer "B.Cu") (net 12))
 (segment (start 88.646 97.536) (end 88.646 100.076) (width 0.2) (layer "B.Cu") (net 12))
 (segment (start 88.646 76.962) (end 88.646 78.74) (width 0.2) (layer "B.Cu") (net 12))
 (segment (start 96.266 105.156) (end 96.266 102.743) (width 0.2) (layer "B.Cu") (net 12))
 (segment (start 88.646 45.974) (end 88.646 48.387) (width 0.2) (layer "B.Cu") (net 12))
 (segment (start 98.806 45.974) (end 94.996 49.784) (width 0.2) (layer "B.Cu") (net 12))
 (segment (start 83.566 88.9) (end 81.026 88.9) (width 0.2) (layer "B.Cu") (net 12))
 (segment (start 86.106 91.44) (end 88.646 88.9) (width 0.2) (layer "B.Cu") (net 12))
 (segment (start 86.106 102.87) (end 86.106 105.156) (width 0.2) (layer "B.Cu") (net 12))
 (segment (start 88.646 102.87) (end 87.376 101.6) (width 0.2) (layer "B.Cu") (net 12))
 (segment (start 93.6625 71.9455) (end 94.488 71.12) (width 0.2) (layer "B.Cu") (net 12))
 (segment (start 83.566 100.33) (end 86.106 102.87) (width 0.2) (layer "B.Cu") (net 12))
 (segment (start 95.123 101.6) (end 84.836 101.6) (width 0.2) (layer "B.Cu") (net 12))
 (segment (start 88.646 48.387) (end 90.043 49.784) (width 0.2) (layer "B.Cu") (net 12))
 (segment (start 94.488 71.12) (end 96.266 71.12) (width 0.2) (layer "B.Cu") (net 12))
 (segment (start 88.646 100.076) (end 87.122 101.6) (width 0.2) (layer "B.Cu") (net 12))
 (segment (start 94.996 49.784) (end 87.376 49.784) (width 0.2) (layer "B.Cu") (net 12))
 (segment (start 93.726 45.974) (end 93.726 46.736) (width 0.2) (layer "B.Cu") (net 12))
 (segment (start 86.106 53.594) (end 86.233 53.594) (width 0.2) (layer "B.Cu") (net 12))
 (segment (start 101.854 96.647) (end 101.854 96.774) (width 0.2) (layer "F.Cu") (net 23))
 (segment (start 99.314 60.96) (end 100.965 62.611) (width 0.2) (layer "F.Cu") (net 23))
 (segment (start 98.806 105.156) (end 101.854 102.108) (width 0.2) (layer "F.Cu") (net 23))
 (segment (start 96.266 91.059) (end 101.854 96.647) (width 0.2) (layer "F.Cu") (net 23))
 (segment (start 101.854 102.108) (end 101.854 96.774) (width 0.2) (layer "F.Cu") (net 23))
 (segment (start 96.266 60.96) (end 99.314 60.96) (width 0.2) (layer "F.Cu") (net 23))
 (via (at 96.266 91.059) (size 0.6) (drill 0.3) (layers "F.Cu" "B.Cu") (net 23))
 (segment (start 98.806 53.594) (end 100.965 55.753) (width 0.2) (layer "B.Cu") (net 23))
 (segment (start 91.567 65.659) (end 91.567 86.487) (width 0.2) (layer "B.Cu") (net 23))
 (segment (start 96.266 60.96) (end 91.567 65.659) (width 0.2) (layer "B.Cu") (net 23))
 (segment (start 96.139 91.059) (end 96.266 91.059) (width 0.2) (layer "B.Cu") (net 23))
 (segment (start 100.965 55.753) (end 100.965 62.611) (width 0.2) (layer "B.Cu") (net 23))
 (segment (start 91.567 86.487) (end 96.139 91.059) (width 0.2) (layer "B.Cu") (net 23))
 (segment (start 100.965 70.231) (end 99.568 68.834) (width 0.2) (layer "B.Cu") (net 26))
 (segment (start 99.568 68.834) (end 99.568 56.896) (width 0.2) (layer "B.Cu") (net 26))
 (segment (start 99.568 56.896) (end 96.266 53.594) (width 0.2) (layer "B.Cu") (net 26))
 (segment (start 100.965 72.771) (end 98.806 74.93) (width 0.2) (layer "B.Cu") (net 24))
 (segment (start 98.806 97.536) (end 98.806 74.93) (width 0.2) (layer "B.Cu") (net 24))
 (segment (start 93.726 97.536) (end 93.726 78.74) (width 0.2) (layer "F.Cu") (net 18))
 (segment (start 93.726 78.74) (end 96.266 76.2) (width 0.2) (layer "F.Cu") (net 18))
 (segment (start 93.326 97.701685) (end 93.506657 97.882343) (width 0.2) (layer "B.Cu") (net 18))
 (segment (start 93.726 55.372) (end 93.726 53.594) (width 0.2) (layer "B.Cu") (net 25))
 (segment (start 96.266 94.869) (end 90.17 88.773) (width 0.2) (layer "B.Cu") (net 25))
 (segment (start 90.17 88.773) (end 90.17 58.928) (width 0.2) (layer "B.Cu") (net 25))
 (segment (start 96.266 97.536) (end 96.266 94.869) (width 0.2) (layer "B.Cu") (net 25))
 (segment (start 90.17 58.928) (end 93.726 55.372) (width 0.2) (layer "B.Cu") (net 25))
 (segment (start 81.026 60.96) (end 84.074 60.96) (width 0.2) (layer "F.Cu") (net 1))
 (segment (start 84.074 60.96) (end 85.725 62.611) (width 0.2) (layer "F.Cu") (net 1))
 (segment (start 84.074 63.5) (end 85.725 65.151) (width 0.2) (layer "F.Cu") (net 2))
 (segment (start 81.026 63.5) (end 84.074 63.5) (width 0.2) (layer "F.Cu") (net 2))
 (segment (start 84.074 66.04) (end 85.725 67.691) (width 0.2) (layer "F.Cu") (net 3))
 (segment (start 81.026 66.04) (end 84.074 66.04) (width 0.2) (layer "F.Cu") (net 3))
 (segment (start 81.026 68.58) (end 84.074 68.58) (width 0.2) (layer "F.Cu") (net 4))
 (segment (start 84.074 68.58) (end 85.725 70.231) (width 0.2) (layer "F.Cu") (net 4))
 (segment (start 84.074 71.12) (end 85.725 72.771) (width 0.2) (layer "F.Cu") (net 5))
 (segment (start 81.026 71.12) (end 84.074 71.12) (width 0.2) (layer "F.Cu") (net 5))
 (segment (start 84.074 73.66) (end 85.725 75.311) (width 0.2) (layer "F.Cu") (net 6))
 (segment (start 81.026 73.66) (end 84.074 73.66) (width 0.2) (layer "F.Cu") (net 6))
 (segment (start 81.026 76.2) (end 84.074 76.2) (width 0.2) (layer "F.Cu") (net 7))
 (segment (start 84.074 76.2) (end 85.725 77.851) (width 0.2) (layer "F.Cu") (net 7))
 (segment (start 84.074 78.74) (end 85.725 80.391) (width 0.2) (layer "F.Cu") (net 8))
 (segment (start 81.026 78.74) (end 84.074 78.74) (width 0.2) (layer "F.Cu") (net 8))
 (segment (start 84.074 81.28) (end 85.725 82.931) (width 0.2) (layer "F.Cu") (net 9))
 (segment (start 81.026 81.28) (end 84.074 81.28) (width 0.2) (layer "F.Cu") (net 9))
 (segment (start 84.074 83.82) (end 85.725 85.471) (width 0.2) (layer "F.Cu") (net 10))
 (segment (start 81.026 83.82) (end 84.074 83.82) (width 0.2) (layer "F.Cu") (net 10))
 (segment (start 81.026 86.36) (end 84.074 86.36) (width 0.2) (layer "F.Cu") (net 11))
 (segment (start 84.074 86.36) (end 85.725 88.011) (width 0.2) (layer "F.Cu") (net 11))
 (segment (start 96.266 63.5) (end 99.314 63.5) (width 0.2) (layer "F.Cu") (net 22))
 (segment (start 99.314 63.5) (end 100.965 65.151) (width 0.2) (layer "F.Cu") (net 22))
 (segment (start 96.266 66.04) (end 99.314 66.04) (width 0.2) (layer "F.Cu") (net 21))
 (segment (start 99.314 66.04) (end 100.965 67.691) (width 0.2) (layer "F.Cu") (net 21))
 (segment (start 96.266 73.66) (end 99.314 73.66) (width 0.2) (layer "F.Cu") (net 19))
 (segment (start 99.314 73.66) (end 100.965 75.311) (width 0.2) (layer "F.Cu") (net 19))
 (segment (start 94.488 70.358) (end 94.488 73.914) (width 0.2) (layer "F.Cu") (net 20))
 (segment (start 94.488 73.914) (end 95.504 74.93) (width 0.2) (layer "F.Cu") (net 20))
 (segment (start 95.504 74.93) (end 98.044 74.93) (width 0.2) (layer "F.Cu") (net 20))
 (segment (start 98.044 74.93) (end 100.965 77.851) (width 0.2) (layer "F.Cu") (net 20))
 (segment (start 96.266 68.58) (end 94.488 70.358) (width 0.2) (layer "F.Cu") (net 20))
 (segment (start 99.314 78.74) (end 100.965 80.391) (width 0.2) (layer "F.Cu") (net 17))
 (segment (start 96.266 78.74) (end 99.314 78.74) (width 0.2) (layer "F.Cu") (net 17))
 (segment (start 99.314 81.28) (end 100.965 82.931) (width 0.2) (layer "F.Cu") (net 16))
 (segment (start 96.266 81.28) (end 99.314 81.28) (width 0.2) (layer "F.Cu") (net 16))
 (segment (start 96.266 83.82) (end 99.314 83.82) (width 0.2) (layer "F.Cu") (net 15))
 (segment (start 99.314 83.82) (end 100.965 85.471) (width 0.2) (layer "F.Cu") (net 15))
 (segment (start 99.314 86.36) (end 100.965 88.011) (width 0.2) (layer "F.Cu") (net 14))
 (segment (start 96.266 86.36) (end 99.314 86.36) (width 0.2) (layer "F.Cu") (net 14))
 (segment (start 99.314 88.9) (end 100.965 90.551) (width 0.2) (layer "F.Cu") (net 13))
 (segment (start 96.266 88.9) (end 99.314 88.9) (width 0.2) (layer "F.Cu") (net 13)))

